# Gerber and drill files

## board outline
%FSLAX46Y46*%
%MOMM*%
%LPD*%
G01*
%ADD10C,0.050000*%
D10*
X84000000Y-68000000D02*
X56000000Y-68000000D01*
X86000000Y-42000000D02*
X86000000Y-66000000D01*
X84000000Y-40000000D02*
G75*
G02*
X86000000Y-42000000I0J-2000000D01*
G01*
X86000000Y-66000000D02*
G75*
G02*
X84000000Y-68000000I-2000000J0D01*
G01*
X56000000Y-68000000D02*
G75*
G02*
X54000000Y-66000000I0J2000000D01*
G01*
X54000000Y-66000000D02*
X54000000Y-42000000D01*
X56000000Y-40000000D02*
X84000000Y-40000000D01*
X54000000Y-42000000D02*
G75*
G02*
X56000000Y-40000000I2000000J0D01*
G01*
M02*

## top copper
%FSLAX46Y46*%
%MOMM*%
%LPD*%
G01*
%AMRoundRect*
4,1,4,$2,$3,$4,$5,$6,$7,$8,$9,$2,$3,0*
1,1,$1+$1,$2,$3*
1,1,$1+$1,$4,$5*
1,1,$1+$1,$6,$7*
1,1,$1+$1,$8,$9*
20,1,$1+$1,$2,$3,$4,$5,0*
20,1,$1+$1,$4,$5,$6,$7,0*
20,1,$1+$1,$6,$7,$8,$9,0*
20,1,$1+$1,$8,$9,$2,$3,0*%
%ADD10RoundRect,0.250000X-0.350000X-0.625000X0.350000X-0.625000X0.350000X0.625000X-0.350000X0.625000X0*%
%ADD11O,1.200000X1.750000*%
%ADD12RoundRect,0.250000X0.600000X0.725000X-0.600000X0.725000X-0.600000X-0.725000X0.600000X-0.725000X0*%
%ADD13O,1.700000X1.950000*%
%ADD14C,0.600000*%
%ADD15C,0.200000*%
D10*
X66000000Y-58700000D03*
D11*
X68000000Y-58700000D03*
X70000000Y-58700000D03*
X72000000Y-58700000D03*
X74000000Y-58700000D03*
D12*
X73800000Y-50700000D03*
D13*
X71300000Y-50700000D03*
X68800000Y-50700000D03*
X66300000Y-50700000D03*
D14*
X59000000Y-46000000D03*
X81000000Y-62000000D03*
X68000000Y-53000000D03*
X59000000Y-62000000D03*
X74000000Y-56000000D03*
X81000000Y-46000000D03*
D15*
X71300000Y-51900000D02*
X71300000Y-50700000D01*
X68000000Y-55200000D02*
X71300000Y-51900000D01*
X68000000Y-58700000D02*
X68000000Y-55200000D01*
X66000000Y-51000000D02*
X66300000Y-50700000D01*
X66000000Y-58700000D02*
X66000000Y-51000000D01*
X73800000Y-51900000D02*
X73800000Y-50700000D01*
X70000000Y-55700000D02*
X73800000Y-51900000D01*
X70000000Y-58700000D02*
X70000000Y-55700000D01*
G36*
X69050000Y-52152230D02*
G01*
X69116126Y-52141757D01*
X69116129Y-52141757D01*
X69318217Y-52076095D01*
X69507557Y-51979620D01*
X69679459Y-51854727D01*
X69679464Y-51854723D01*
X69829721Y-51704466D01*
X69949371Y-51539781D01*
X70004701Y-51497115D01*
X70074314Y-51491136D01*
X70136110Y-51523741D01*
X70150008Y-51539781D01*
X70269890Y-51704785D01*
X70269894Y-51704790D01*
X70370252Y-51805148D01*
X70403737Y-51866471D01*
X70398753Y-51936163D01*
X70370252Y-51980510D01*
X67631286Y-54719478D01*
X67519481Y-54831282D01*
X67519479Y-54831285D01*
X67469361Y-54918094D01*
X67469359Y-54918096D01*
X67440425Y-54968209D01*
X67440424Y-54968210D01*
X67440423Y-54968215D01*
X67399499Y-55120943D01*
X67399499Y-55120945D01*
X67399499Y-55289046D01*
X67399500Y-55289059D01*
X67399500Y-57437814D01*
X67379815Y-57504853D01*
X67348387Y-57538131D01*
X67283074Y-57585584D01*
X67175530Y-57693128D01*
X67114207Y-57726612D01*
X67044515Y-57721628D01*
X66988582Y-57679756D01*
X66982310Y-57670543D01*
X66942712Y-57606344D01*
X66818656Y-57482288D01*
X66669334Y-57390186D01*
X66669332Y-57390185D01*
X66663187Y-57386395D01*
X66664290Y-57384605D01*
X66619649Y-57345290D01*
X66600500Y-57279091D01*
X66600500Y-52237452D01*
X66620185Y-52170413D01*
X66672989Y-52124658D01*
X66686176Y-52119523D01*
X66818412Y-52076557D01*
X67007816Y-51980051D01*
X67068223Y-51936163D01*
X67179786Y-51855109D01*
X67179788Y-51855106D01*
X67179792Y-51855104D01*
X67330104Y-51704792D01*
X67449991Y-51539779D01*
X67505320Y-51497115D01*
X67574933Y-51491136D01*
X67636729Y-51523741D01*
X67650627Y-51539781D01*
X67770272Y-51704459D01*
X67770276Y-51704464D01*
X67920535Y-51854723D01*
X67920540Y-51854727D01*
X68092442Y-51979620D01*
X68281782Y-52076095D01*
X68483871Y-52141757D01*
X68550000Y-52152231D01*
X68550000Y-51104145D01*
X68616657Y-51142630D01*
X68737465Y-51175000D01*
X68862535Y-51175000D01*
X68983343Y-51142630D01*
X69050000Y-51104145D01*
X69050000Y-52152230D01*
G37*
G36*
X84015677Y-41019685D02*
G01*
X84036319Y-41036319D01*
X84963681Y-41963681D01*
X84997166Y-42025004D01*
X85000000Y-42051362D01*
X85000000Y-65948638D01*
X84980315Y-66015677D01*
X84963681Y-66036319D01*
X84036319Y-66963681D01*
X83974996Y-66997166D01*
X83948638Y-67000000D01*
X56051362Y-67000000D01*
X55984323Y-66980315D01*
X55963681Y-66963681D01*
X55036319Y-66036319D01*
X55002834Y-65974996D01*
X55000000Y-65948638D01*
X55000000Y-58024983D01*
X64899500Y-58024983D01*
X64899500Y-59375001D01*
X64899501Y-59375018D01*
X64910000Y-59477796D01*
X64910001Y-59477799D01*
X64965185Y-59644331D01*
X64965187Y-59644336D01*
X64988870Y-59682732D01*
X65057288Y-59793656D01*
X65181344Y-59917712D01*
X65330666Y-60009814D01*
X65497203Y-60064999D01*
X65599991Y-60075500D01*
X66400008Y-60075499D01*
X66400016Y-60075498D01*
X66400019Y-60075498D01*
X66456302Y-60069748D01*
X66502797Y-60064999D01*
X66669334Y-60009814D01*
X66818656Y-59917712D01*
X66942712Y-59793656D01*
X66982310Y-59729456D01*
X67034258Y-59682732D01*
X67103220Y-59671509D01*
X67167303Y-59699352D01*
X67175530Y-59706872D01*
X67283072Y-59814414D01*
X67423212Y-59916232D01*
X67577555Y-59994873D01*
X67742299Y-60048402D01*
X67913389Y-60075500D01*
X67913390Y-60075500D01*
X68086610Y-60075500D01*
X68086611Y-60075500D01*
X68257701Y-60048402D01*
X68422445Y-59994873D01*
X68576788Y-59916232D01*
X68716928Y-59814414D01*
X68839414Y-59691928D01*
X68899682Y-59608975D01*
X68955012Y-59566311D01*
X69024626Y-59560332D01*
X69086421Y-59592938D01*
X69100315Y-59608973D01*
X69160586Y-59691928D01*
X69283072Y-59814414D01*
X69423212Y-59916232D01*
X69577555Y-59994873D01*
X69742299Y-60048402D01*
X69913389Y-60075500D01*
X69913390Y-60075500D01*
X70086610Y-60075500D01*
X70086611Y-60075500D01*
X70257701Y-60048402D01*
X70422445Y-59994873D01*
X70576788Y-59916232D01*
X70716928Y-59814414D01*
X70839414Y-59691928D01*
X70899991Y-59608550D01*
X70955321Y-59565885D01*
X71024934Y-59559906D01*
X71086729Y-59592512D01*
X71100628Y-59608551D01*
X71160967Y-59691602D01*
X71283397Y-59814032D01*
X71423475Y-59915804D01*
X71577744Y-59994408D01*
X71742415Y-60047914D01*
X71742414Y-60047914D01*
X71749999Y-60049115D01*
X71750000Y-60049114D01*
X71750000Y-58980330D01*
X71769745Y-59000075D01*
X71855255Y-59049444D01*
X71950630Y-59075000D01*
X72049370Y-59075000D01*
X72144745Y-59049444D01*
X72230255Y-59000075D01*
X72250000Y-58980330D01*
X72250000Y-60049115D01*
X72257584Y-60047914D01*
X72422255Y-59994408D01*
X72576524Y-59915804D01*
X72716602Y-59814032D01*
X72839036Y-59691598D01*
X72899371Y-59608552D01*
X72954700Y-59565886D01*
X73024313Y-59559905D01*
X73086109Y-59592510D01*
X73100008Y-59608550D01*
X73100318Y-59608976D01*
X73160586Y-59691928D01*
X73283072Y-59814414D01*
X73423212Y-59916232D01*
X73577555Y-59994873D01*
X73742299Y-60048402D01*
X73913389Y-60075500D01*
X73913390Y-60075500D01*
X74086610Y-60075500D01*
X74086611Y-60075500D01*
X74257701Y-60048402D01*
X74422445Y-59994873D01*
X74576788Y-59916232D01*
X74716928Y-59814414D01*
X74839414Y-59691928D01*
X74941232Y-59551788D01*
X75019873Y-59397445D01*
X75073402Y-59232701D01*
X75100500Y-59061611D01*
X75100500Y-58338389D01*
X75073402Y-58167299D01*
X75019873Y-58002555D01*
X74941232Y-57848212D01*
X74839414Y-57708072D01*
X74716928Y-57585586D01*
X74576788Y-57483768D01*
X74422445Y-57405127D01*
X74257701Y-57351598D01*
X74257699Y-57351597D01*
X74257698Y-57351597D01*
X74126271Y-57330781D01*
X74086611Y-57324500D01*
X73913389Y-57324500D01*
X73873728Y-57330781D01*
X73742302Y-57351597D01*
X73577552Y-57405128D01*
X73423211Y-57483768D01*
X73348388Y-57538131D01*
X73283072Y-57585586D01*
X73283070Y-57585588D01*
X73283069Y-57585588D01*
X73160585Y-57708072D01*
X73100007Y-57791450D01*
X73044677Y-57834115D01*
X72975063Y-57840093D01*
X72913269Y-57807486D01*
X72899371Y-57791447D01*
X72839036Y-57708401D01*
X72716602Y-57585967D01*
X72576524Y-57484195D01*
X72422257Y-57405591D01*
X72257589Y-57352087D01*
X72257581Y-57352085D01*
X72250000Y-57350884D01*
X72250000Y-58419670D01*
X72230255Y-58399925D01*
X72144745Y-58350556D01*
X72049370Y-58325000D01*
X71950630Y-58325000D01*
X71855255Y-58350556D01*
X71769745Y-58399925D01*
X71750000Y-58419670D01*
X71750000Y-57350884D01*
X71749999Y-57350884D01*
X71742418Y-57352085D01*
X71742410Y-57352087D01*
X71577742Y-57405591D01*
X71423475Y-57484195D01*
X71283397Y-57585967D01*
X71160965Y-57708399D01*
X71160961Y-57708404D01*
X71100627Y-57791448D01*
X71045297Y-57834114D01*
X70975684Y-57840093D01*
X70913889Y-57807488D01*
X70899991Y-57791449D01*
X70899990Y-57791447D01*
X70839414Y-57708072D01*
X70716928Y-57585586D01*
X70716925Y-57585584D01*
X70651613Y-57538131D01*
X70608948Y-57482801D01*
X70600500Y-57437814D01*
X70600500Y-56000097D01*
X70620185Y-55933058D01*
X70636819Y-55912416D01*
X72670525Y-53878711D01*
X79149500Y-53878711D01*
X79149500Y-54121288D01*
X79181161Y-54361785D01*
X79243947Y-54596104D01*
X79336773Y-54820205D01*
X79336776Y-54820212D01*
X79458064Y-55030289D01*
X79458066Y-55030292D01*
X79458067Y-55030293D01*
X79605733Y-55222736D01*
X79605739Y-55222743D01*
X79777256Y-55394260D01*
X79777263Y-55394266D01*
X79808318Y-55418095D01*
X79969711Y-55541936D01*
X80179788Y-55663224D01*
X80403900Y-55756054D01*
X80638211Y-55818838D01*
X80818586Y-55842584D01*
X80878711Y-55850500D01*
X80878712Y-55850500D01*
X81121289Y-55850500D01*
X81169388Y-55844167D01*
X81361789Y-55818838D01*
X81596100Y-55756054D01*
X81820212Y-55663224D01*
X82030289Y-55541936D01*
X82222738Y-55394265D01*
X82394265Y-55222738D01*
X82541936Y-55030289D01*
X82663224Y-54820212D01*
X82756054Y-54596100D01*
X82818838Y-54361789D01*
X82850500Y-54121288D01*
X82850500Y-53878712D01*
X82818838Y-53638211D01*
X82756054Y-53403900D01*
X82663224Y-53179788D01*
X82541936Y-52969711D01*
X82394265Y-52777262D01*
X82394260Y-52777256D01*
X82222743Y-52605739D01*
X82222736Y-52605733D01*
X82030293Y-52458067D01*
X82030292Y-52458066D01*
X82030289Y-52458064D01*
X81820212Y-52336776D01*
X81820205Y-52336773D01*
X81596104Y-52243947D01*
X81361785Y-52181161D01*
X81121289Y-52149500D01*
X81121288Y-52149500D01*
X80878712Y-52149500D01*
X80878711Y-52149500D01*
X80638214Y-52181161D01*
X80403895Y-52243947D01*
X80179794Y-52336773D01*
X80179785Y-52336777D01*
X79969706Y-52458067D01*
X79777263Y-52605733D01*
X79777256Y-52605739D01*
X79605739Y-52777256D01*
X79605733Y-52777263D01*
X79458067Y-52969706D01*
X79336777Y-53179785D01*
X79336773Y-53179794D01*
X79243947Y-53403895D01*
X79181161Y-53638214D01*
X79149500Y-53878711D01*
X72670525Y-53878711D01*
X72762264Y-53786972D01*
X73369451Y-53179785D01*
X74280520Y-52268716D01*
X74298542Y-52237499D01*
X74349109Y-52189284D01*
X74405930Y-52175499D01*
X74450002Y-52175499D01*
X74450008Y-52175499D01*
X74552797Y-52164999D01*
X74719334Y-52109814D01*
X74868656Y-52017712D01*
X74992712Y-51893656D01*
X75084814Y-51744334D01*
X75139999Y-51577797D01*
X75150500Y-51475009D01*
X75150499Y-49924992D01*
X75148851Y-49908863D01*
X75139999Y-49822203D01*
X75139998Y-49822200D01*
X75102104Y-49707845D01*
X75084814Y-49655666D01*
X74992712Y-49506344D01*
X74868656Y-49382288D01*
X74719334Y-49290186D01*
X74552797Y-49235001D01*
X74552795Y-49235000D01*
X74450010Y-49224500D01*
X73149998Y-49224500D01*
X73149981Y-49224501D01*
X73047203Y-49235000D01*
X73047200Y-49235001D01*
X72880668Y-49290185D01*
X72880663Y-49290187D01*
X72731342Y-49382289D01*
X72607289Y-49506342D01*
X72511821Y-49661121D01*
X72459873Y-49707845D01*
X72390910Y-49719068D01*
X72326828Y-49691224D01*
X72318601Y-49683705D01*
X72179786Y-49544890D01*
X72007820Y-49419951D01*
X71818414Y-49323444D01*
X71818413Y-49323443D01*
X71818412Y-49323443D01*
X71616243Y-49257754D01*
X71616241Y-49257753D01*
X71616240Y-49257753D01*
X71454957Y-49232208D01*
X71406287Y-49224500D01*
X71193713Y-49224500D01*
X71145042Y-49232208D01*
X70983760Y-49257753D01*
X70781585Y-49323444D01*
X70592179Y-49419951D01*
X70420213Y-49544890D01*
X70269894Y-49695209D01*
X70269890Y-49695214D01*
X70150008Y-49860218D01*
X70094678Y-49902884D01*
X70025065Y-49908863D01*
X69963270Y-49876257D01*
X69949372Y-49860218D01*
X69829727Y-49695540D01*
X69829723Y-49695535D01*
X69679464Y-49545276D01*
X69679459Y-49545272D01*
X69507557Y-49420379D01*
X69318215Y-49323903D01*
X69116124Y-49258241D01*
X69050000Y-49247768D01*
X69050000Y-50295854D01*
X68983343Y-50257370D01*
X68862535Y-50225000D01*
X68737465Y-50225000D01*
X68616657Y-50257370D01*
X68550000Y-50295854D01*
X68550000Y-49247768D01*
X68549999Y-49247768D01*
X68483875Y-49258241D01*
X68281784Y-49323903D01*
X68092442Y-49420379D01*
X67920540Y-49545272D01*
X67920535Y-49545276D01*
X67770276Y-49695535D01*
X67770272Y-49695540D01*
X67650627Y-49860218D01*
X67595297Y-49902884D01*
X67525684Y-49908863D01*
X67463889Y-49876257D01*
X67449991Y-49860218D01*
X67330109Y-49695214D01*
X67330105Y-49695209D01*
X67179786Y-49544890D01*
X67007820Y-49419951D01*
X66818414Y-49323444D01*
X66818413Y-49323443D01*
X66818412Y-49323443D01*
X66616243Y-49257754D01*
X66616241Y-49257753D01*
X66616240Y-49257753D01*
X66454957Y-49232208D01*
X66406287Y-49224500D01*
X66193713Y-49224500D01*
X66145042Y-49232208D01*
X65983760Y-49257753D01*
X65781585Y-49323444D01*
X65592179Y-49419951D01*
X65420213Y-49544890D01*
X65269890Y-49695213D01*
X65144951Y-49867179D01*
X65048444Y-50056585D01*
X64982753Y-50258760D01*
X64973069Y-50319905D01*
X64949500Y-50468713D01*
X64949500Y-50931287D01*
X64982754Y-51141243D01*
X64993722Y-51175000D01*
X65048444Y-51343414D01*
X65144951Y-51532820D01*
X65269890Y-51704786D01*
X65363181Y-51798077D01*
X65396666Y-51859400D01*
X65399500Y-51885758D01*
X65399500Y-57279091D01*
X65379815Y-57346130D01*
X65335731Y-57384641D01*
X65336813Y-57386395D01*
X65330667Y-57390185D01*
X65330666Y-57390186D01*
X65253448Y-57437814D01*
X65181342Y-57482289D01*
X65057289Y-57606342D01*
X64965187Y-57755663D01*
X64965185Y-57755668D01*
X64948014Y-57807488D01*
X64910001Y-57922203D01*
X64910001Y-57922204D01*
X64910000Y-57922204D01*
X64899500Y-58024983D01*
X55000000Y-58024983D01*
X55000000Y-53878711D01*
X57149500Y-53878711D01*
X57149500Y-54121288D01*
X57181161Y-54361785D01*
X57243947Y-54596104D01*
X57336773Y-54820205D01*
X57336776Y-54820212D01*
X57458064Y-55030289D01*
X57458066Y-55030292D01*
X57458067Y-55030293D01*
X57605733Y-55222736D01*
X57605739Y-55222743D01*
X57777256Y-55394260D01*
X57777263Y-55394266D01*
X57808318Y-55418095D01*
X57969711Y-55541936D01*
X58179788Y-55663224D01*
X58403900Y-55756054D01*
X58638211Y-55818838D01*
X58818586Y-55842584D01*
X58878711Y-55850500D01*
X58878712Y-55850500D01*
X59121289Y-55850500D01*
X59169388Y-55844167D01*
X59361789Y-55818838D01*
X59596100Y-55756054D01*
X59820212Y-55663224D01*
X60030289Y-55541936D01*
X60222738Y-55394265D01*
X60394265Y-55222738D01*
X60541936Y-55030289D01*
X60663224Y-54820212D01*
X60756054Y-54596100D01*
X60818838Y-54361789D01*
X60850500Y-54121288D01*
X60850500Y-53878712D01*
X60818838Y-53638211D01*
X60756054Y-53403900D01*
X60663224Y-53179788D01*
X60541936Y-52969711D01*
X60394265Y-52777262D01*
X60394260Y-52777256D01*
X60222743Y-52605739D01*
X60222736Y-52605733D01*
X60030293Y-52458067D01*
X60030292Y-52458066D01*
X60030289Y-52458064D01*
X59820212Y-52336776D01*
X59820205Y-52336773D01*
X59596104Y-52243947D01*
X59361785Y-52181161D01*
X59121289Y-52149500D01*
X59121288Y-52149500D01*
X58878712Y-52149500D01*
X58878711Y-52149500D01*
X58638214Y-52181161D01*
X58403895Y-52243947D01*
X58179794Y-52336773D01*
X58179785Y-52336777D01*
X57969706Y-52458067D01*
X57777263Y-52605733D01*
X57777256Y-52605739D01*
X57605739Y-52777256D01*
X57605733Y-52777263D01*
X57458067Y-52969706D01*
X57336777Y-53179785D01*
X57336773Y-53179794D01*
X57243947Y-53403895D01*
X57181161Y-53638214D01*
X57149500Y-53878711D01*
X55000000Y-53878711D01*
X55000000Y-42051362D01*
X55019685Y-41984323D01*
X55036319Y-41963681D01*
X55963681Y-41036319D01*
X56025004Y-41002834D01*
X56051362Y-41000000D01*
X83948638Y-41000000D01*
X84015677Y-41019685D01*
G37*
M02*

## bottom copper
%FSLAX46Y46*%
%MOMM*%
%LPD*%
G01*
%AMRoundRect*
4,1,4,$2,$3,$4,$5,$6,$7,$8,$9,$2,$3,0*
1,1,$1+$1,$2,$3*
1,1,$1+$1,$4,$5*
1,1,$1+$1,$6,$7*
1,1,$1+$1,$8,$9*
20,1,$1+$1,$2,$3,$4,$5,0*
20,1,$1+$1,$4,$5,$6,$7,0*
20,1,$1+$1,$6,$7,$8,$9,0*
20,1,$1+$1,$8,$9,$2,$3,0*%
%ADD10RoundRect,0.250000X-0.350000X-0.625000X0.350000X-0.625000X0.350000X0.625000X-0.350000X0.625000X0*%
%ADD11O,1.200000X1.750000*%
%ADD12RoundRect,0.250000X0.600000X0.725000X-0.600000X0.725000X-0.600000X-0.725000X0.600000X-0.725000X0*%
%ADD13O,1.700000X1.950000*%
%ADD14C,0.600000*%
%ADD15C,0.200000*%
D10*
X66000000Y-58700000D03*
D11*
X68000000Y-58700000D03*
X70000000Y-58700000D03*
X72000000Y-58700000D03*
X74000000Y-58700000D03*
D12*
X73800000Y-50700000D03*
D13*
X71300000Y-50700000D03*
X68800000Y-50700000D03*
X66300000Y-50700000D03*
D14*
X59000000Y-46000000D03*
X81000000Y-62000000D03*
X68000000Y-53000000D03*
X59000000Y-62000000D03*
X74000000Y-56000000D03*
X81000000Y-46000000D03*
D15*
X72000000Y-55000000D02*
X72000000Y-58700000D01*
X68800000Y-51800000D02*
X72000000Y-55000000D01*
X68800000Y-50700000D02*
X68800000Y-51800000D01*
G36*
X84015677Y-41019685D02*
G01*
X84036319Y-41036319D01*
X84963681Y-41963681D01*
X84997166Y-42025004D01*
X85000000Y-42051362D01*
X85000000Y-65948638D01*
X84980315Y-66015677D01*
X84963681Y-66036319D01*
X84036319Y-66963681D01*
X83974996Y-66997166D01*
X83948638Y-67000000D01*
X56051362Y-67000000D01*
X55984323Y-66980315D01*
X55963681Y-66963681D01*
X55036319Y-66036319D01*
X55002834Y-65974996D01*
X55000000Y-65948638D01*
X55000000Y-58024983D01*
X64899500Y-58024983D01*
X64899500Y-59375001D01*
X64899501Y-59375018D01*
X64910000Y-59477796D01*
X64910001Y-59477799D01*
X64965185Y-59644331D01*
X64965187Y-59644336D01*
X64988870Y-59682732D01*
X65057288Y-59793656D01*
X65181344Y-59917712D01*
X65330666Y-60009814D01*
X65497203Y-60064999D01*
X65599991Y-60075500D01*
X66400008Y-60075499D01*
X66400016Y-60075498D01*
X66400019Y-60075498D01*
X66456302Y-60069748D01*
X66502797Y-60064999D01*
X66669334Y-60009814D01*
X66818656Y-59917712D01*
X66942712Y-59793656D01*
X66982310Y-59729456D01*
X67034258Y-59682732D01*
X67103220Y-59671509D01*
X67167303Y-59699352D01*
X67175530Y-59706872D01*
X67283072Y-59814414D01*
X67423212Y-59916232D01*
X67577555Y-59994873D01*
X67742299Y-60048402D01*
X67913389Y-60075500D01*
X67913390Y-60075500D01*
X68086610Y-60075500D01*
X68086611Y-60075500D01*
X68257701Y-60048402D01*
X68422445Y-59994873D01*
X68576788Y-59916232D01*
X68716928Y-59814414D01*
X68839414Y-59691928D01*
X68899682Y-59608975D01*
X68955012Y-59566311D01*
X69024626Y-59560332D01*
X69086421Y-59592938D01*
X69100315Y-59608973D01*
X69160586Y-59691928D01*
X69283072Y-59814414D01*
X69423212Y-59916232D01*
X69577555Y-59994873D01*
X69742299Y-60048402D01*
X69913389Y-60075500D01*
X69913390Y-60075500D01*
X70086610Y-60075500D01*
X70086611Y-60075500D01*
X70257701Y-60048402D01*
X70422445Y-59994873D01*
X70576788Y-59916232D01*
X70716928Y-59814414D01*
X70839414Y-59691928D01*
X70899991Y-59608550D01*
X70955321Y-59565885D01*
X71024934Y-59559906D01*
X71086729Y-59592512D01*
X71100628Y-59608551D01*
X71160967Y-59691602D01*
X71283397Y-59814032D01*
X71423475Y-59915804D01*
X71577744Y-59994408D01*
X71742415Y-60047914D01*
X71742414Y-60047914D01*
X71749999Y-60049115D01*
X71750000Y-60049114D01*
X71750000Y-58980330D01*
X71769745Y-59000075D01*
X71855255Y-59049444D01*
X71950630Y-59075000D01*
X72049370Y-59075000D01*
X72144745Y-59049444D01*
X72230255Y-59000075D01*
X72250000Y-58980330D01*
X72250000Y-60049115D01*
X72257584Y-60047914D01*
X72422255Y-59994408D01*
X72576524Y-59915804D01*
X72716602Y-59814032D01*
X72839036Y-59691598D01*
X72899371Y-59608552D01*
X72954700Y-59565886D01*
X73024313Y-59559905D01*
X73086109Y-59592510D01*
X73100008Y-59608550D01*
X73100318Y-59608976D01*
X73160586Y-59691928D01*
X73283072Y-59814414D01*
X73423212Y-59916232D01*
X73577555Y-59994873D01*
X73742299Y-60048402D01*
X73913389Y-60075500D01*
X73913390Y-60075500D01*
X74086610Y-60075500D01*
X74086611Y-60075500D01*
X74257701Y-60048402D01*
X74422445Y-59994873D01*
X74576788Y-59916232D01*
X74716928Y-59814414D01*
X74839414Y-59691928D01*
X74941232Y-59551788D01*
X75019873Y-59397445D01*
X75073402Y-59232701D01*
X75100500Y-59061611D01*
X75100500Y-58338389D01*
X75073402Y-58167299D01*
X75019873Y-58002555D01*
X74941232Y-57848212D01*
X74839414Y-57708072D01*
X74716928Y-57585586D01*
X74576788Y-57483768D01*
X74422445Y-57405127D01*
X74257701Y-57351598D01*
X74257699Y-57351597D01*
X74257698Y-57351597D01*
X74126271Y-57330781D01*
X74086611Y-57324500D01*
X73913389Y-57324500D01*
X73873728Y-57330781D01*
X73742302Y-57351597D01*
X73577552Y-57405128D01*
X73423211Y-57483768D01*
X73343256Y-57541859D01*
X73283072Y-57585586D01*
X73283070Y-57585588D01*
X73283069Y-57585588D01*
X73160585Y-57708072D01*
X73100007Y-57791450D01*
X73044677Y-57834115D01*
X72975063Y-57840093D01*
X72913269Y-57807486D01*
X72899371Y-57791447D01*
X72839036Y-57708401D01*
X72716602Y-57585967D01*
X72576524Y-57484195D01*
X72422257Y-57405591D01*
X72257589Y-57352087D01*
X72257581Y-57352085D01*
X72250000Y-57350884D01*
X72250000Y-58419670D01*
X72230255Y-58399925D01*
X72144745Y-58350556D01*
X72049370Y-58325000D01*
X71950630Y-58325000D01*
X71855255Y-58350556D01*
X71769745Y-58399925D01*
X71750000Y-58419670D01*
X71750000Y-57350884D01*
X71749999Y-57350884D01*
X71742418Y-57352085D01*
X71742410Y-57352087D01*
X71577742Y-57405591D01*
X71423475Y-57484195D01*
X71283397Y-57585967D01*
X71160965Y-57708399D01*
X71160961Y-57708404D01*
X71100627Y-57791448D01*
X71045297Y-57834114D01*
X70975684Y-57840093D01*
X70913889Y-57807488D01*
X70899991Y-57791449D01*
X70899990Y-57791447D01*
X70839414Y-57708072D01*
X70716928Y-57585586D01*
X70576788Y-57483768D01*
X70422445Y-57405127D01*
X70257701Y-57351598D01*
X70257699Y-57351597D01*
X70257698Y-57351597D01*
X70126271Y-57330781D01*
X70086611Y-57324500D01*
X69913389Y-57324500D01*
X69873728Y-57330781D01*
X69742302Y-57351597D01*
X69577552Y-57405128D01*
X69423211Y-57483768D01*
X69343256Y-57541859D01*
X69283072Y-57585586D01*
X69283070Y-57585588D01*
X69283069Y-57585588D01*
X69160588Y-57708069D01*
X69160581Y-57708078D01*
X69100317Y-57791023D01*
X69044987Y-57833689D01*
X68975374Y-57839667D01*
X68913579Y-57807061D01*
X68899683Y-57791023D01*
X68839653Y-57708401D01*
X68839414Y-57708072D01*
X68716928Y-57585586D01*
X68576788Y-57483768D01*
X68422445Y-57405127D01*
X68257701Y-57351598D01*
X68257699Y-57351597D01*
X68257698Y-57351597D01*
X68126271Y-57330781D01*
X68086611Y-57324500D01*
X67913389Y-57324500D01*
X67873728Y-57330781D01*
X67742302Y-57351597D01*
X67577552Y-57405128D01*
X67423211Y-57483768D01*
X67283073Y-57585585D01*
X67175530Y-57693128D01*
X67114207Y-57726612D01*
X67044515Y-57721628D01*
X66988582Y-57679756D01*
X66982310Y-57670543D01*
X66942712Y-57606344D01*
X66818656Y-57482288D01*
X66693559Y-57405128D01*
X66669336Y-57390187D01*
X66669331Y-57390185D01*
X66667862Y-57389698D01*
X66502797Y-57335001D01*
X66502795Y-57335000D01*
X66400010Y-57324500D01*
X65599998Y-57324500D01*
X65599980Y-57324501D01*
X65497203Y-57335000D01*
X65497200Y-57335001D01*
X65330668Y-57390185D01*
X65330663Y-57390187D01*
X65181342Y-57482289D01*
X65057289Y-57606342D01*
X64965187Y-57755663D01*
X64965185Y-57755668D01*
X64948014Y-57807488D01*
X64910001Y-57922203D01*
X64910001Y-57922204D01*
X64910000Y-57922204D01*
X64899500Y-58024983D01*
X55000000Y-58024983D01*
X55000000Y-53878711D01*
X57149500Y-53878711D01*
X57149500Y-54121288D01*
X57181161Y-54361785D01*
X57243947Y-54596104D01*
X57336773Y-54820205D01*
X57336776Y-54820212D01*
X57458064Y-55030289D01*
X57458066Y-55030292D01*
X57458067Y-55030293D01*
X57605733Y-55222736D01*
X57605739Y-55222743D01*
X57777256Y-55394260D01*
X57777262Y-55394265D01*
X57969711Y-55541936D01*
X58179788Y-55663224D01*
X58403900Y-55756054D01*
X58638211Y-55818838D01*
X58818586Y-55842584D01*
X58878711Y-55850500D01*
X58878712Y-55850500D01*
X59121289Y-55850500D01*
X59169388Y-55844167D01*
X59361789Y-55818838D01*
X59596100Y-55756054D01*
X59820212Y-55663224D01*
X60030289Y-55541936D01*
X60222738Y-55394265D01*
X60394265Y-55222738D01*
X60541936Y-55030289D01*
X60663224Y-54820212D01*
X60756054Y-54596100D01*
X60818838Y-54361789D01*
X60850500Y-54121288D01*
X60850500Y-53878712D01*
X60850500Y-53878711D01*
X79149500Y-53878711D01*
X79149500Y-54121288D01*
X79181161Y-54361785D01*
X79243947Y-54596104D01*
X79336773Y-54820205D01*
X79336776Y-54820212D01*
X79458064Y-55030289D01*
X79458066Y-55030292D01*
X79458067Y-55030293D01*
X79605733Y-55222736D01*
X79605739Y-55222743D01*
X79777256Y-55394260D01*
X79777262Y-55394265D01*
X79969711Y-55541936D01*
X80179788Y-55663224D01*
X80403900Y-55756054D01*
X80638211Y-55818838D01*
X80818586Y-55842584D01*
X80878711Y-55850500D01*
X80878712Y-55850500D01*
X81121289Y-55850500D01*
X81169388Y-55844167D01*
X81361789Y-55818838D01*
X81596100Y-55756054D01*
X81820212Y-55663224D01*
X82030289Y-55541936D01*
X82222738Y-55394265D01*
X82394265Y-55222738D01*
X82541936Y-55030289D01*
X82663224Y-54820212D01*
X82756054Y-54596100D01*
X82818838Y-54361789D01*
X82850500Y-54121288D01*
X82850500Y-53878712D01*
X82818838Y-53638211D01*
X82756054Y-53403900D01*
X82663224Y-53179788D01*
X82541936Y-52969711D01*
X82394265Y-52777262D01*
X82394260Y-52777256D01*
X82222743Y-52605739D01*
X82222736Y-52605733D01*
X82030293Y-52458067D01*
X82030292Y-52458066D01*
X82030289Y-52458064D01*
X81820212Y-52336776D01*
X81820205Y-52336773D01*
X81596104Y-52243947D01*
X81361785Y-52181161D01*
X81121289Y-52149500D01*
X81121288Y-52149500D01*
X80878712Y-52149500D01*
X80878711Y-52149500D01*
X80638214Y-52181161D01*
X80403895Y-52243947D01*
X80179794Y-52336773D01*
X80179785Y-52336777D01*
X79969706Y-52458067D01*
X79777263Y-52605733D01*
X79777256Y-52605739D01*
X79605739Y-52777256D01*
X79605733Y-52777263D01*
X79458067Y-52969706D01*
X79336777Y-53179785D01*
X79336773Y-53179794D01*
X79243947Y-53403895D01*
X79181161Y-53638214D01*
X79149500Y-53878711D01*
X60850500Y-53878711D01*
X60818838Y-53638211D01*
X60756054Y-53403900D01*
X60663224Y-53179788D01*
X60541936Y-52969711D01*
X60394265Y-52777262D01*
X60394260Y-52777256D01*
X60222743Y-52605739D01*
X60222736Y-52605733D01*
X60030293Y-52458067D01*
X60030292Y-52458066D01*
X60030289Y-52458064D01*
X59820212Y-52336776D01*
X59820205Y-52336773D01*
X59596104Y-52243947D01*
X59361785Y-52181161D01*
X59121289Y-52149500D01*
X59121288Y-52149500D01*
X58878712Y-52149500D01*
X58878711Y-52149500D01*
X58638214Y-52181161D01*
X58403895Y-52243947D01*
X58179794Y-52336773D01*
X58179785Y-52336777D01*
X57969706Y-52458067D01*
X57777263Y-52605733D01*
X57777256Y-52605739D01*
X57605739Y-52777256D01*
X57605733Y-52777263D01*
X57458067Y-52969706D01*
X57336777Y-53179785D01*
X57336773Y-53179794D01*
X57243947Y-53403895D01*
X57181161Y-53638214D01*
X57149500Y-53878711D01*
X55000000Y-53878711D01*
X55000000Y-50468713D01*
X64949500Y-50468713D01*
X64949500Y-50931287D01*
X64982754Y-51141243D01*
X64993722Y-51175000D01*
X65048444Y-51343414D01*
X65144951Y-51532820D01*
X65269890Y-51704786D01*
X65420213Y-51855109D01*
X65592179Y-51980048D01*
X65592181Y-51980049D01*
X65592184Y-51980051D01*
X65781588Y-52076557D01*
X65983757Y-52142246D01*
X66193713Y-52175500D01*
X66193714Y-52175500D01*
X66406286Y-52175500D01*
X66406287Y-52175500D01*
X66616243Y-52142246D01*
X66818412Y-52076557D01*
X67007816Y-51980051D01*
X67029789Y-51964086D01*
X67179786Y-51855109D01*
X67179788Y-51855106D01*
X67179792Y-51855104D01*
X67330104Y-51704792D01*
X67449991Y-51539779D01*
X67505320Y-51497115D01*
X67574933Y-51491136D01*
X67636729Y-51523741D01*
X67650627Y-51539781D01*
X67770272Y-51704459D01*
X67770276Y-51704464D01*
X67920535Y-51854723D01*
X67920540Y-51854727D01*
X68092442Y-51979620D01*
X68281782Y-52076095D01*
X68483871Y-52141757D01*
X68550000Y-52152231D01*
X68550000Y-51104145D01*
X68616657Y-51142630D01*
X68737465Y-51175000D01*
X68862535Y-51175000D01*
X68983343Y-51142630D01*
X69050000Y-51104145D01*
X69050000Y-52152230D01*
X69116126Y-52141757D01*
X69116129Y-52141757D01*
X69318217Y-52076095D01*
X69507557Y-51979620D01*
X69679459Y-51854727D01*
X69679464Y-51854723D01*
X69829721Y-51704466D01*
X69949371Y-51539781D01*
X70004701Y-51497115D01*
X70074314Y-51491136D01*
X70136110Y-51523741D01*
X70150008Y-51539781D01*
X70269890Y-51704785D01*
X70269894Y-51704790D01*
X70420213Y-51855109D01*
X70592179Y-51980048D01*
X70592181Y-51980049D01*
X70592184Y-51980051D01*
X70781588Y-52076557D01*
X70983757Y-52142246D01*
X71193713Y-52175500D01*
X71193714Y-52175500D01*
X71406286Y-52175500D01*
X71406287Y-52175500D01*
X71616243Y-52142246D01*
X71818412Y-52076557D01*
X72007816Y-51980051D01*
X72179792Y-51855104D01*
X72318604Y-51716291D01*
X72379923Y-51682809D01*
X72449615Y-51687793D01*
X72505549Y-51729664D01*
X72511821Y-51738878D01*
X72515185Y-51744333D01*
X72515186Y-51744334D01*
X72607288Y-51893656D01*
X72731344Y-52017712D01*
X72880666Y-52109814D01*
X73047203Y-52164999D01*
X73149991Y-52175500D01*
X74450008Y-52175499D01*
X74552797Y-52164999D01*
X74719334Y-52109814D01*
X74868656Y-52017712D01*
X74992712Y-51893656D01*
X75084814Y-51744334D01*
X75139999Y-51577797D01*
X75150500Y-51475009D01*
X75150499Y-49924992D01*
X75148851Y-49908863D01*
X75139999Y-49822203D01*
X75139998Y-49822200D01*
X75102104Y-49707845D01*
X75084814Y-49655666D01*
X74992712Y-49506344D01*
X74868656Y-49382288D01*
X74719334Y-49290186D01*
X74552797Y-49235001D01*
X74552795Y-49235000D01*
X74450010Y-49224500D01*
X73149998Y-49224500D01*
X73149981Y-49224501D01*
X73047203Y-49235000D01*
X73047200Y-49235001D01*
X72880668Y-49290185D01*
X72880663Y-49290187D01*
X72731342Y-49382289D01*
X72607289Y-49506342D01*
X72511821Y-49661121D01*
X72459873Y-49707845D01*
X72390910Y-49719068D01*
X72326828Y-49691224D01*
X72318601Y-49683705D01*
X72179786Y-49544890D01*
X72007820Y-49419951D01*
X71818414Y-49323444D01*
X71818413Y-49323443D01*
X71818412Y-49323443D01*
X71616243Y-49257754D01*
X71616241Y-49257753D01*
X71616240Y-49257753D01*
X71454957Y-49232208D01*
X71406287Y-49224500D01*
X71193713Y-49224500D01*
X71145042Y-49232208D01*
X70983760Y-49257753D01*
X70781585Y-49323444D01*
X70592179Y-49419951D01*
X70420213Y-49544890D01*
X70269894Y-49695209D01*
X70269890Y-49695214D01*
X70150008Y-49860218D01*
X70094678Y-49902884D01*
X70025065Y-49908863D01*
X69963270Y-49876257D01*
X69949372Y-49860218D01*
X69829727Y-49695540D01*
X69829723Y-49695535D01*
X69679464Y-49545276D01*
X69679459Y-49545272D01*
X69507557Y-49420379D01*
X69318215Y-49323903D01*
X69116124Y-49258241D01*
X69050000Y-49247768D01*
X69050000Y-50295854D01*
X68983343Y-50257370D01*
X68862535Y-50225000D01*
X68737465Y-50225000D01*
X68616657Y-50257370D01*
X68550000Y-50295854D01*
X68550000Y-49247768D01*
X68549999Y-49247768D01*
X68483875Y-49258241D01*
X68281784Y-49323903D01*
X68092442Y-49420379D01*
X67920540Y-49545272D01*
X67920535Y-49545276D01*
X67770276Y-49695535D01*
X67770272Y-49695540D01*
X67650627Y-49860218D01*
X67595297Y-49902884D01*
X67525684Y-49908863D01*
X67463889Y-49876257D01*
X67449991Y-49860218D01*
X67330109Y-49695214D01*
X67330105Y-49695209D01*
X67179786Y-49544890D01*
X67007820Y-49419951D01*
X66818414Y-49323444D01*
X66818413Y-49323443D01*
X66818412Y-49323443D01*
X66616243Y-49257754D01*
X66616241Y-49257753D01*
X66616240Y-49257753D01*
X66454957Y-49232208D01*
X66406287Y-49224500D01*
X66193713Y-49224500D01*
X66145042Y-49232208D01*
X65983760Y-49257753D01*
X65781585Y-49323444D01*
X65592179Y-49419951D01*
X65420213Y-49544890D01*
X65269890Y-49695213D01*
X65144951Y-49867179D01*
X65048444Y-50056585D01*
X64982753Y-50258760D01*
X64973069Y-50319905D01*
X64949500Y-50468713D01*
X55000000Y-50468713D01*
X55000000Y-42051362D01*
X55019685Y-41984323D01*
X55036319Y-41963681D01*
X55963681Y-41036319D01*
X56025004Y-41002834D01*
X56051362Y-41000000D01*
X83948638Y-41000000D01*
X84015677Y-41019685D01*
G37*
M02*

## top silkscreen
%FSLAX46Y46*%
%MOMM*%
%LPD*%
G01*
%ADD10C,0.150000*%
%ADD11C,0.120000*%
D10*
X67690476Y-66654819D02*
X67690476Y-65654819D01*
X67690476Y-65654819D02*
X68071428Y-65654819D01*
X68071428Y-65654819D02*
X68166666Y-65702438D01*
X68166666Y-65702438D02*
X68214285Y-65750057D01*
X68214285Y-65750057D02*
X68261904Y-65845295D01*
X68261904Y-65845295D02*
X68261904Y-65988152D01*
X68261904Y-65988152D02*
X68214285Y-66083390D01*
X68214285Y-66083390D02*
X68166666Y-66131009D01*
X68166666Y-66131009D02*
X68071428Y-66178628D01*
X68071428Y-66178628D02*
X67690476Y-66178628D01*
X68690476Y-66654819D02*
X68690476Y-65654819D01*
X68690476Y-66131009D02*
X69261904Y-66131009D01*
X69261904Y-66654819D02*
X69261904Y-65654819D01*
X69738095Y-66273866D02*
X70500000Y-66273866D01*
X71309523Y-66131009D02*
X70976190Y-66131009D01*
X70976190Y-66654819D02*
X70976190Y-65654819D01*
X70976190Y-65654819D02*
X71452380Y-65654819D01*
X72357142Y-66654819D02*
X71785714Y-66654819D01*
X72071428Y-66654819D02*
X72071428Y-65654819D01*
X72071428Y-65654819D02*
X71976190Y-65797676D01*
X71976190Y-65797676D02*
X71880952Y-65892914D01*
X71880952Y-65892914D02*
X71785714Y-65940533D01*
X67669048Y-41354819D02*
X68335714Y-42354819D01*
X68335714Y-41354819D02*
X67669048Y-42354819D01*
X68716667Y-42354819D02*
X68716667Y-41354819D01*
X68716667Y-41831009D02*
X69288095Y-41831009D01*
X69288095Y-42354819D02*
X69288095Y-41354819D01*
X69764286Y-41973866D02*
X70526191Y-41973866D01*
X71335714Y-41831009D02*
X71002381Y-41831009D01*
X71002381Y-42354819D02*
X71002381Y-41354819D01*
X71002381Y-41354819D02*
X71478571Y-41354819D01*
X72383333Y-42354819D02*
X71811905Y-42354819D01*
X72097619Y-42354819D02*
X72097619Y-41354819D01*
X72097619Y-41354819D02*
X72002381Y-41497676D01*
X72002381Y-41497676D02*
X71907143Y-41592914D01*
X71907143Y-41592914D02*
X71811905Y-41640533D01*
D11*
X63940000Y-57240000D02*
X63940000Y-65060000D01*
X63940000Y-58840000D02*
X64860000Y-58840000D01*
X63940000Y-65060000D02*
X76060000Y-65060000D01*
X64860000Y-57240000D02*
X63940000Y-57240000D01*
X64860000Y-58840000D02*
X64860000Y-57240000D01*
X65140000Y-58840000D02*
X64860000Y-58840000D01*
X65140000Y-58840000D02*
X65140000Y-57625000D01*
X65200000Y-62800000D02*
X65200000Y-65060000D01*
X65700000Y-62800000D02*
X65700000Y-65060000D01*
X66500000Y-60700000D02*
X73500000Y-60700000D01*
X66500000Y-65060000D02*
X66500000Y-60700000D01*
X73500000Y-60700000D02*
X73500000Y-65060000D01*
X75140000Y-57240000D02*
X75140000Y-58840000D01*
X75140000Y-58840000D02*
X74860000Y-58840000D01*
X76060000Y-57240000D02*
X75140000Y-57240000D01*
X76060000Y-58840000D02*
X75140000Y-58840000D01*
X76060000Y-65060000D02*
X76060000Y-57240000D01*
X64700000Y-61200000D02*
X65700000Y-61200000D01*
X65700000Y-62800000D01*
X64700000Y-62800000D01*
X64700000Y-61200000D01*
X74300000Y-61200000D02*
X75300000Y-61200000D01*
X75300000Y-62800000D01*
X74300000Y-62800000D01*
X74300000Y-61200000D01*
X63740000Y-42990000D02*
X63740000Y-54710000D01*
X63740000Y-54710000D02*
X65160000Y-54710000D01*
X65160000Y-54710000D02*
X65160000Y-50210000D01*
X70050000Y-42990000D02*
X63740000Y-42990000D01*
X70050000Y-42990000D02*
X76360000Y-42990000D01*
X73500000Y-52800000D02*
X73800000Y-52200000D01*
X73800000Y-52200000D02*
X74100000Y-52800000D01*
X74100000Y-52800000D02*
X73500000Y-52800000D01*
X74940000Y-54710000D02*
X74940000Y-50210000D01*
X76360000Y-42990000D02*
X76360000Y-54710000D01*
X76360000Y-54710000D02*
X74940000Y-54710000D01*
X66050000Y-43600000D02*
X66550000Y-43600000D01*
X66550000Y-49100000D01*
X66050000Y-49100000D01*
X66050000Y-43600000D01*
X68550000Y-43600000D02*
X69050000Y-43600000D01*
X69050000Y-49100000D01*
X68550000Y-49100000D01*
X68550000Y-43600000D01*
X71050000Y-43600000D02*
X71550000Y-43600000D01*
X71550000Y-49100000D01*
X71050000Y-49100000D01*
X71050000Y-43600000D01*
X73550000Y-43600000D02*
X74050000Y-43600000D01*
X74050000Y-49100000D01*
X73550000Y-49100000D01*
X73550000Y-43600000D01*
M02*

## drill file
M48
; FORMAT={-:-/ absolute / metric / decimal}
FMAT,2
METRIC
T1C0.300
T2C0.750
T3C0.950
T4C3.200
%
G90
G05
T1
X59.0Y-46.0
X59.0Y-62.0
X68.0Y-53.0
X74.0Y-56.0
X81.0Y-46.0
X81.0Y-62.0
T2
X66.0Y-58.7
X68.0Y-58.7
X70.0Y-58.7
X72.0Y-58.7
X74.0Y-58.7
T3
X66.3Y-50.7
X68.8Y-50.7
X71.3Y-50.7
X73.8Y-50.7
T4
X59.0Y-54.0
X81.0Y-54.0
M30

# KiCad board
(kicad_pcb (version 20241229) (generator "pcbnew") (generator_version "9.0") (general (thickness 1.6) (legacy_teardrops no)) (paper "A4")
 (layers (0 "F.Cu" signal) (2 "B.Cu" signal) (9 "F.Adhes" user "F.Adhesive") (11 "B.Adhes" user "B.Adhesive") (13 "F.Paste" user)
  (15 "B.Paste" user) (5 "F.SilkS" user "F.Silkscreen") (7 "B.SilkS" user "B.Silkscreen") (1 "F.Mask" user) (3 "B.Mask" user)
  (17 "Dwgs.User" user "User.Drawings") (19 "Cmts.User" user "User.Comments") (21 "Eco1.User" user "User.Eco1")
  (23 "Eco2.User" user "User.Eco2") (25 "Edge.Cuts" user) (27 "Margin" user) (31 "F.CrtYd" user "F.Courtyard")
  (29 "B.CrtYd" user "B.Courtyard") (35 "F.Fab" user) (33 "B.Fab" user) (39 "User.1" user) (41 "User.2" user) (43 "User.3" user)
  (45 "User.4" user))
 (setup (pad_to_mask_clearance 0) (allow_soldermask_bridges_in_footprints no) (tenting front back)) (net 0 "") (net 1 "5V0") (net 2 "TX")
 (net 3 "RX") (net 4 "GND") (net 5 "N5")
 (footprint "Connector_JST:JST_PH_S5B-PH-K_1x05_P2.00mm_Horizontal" (layer "F.Cu") (at 66 58.7)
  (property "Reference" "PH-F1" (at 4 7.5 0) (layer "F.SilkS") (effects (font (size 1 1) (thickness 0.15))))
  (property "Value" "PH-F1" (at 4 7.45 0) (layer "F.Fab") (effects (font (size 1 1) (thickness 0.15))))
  (fp_line (start -2.06 -1.46) (end -2.06 6.36) (stroke (width 0.12) (type solid)) (layer "F.SilkS"))
  (fp_line (start -2.06 0.14) (end -1.14 0.14) (stroke (width 0.12) (type solid)) (layer "F.SilkS"))
  (fp_line (start -2.06 6.36) (end 10.06 6.36) (stroke (width 0.12) (type solid)) (layer "F.SilkS"))
  (fp_line (start -1.14 -1.46) (end -2.06 -1.46) (stroke (width 0.12) (type solid)) (layer "F.SilkS"))
  (fp_line (start -1.14 0.14) (end -1.14 -1.46) (stroke (width 0.12) (type solid)) (layer "F.SilkS"))
  (fp_line (start -0.86 0.14) (end -1.14 0.14) (stroke (width 0.12) (type solid)) (layer "F.SilkS"))
  (fp_line (start -0.86 0.14) (end -0.86 -1.075) (stroke (width 0.12) (type solid)) (layer "F.SilkS"))
  (fp_line (start -0.8 4.1) (end -0.8 6.36) (stroke (width 0.12) (type solid)) (layer "F.SilkS"))
  (fp_line (start -0.3 4.1) (end -0.3 6.36) (stroke (width 0.12) (type solid)) (layer "F.SilkS"))
  (fp_line (start 0.5 2) (end 7.5 2) (stroke (width 0.12) (type solid)) (layer "F.SilkS"))
  (fp_line (start 0.5 6.36) (end 0.5 2) (stroke (width 0.12) (type solid)) (layer "F.SilkS"))
  (fp_line (start 7.5 2) (end 7.5 6.36) (stroke (width 0.12) (type solid)) (layer "F.SilkS"))
  (fp_line (start 9.14 -1.46) (end 9.14 0.14) (stroke (width 0.12) (type solid)) (layer "F.SilkS"))
  (fp_line (start 9.14 0.14) (end 8.86 0.14) (stroke (width 0.12) (type solid)) (layer "F.SilkS"))
  (fp_line (start 10.06 -1.46) (end 9.14 -1.46) (stroke (width 0.12) (type solid)) (layer "F.SilkS"))
  (fp_line (start 10.06 0.14) (end 9.14 0.14) (stroke (width 0.12) (type solid)) (layer "F.SilkS"))
  (fp_line (start 10.06 6.36) (end 10.06 -1.46) (stroke (width 0.12) (type solid)) (layer "F.SilkS"))
  (fp_rect (start -1.3 2.5) (end -0.3 4.1) (stroke (width 0.12) (type solid)) (fill no) (layer "F.SilkS"))
  (fp_rect (start 8.3 2.5) (end 9.3 4.1) (stroke (width 0.12) (type solid)) (fill no) (layer "F.SilkS"))
  (pad "1" thru_hole roundrect (at 0 0) (size 1.2 1.75) (drill 0.75) (layers "*.Cu" "*.Mask") (remove_unused_layers no)
   (roundrect_rratio 0.208333) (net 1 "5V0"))
  (pad "2" thru_hole oval (at 2 0) (size 1.2 1.75) (drill 0.75) (layers "*.Cu" "*.Mask") (remove_unused_layers no) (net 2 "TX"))
  (pad "3" thru_hole oval (at 4 0) (size 1.2 1.75) (drill 0.75) (layers "*.Cu" "*.Mask") (remove_unused_layers no) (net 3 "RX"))
  (pad "4" thru_hole oval (at 6 0) (size 1.2 1.75) (drill 0.75) (layers "*.Cu" "*.Mask") (remove_unused_layers no) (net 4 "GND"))
  (pad "5" thru_hole oval (at 8 0) (size 1.2 1.75) (drill 0.75) (layers "*.Cu" "*.Mask") (remove_unused_layers no) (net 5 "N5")))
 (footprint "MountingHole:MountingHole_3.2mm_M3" (layer "F.Cu") (at 59 54)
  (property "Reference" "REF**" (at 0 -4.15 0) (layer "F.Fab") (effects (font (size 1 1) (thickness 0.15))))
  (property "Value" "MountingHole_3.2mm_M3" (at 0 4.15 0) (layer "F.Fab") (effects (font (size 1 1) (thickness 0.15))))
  (pad "" np_thru_hole circle (at 0 0) (size 3.2 3.2) (drill 3.2) (layers "*.Cu" "*.Mask")))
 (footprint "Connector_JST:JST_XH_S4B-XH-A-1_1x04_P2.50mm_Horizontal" (layer "F.Cu") (at 73.8 50.7 180)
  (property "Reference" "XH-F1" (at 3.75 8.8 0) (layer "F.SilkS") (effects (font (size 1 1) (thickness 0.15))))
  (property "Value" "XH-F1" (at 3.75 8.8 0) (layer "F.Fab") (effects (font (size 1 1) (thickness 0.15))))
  (fp_line (start 10.06 7.71) (end 10.06 -4.01) (stroke (width 0.12) (type solid)) (layer "F.SilkS"))
  (fp_line (start 10.06 -4.01) (end 8.64 -4.01) (stroke (width 0.12) (type solid)) (layer "F.SilkS"))
  (fp_line (start 8.64 -4.01) (end 8.64 0.49) (stroke (width 0.12) (type solid)) (layer "F.SilkS"))
  (fp_line (start 3.75 7.71) (end 10.06 7.71) (stroke (width 0.12) (type solid)) (layer "F.SilkS"))
  (fp_line (start 3.75 7.71) (end -2.56 7.71) (stroke (width 0.12) (type solid)) (layer "F.SilkS"))
  (fp_line (start 0.3 -2.1) (end 0 -1.5) (stroke (width 0.12) (type solid)) (layer "F.SilkS"))
  (fp_line (start 0 -1.5) (end -0.3 -2.1) (stroke (width 0.12) (type solid)) (layer "F.SilkS"))
  (fp_line (start -0.3 -2.1) (end 0.3 -2.1) (stroke (width 0.12) (type solid)) (layer "F.SilkS"))
  (fp_line (start -1.14 -4.01) (end -1.14 0.49) (stroke (width 0.12) (type solid)) (layer "F.SilkS"))
  (fp_line (start -2.56 7.71) (end -2.56 -4.01) (stroke (width 0.12) (type solid)) (layer "F.SilkS"))
  (fp_line (start -2.56 -4.01) (end -1.14 -4.01) (stroke (width 0.12) (type solid)) (layer "F.SilkS"))
  (fp_rect (start 7.25 1.6) (end 7.75 7.1) (stroke (width 0.12) (type solid)) (fill no) (layer "F.SilkS"))
  (fp_rect (start 4.75 1.6) (end 5.25 7.1) (stroke (width 0.12) (type solid)) (fill no) (layer "F.SilkS"))
  (fp_rect (start 2.25 1.6) (end 2.75 7.1) (stroke (width 0.12) (type solid)) (fill no) (layer "F.SilkS"))
  (fp_rect (start -0.25 1.6) (end 0.25 7.1) (stroke (width 0.12) (type solid)) (fill no) (layer "F.SilkS"))
  (pad "1" thru_hole roundrect (at 0 0 180) (size 1.7 1.95) (drill 0.95) (layers "*.Cu" "*.Mask") (remove_unused_layers no)
   (roundrect_rratio 0.147059) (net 3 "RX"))
  (pad "2" thru_hole oval (at 2.5 0 180) (size 1.7 1.95) (drill 0.95) (layers "*.Cu" "*.Mask") (remove_unused_layers no) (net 2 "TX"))
  (pad "3" thru_hole oval (at 5 0 180) (size 1.7 1.95) (drill 0.95) (layers "*.Cu" "*.Mask") (remove_unused_layers no) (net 4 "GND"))
  (pad "4" thru_hole oval (at 7.5 0 180) (size 1.7 1.95) (drill 0.95) (layers "*.Cu" "*.Mask") (remove_unused_layers no) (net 1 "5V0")))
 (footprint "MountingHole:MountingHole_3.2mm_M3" (layer "F.Cu") (at 81 54)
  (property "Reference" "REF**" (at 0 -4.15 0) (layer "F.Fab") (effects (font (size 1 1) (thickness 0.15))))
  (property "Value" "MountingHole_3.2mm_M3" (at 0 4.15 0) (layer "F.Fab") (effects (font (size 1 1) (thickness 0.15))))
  (pad "" np_thru_hole circle (at 0 0) (size 3.2 3.2) (drill 3.2) (layers "*.Cu" "*.Mask")))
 (gr_line (start 84 68) (end 56 68) (stroke (width 0.05) (type default)) (layer "Edge.Cuts"))
 (gr_line (start 86 42) (end 86 66) (stroke (width 0.05) (type default)) (layer "Edge.Cuts"))
 (gr_arc (start 84 40) (mid 85.414214 40.585786) (end 86 42) (stroke (width 0.05) (type default)) (layer "Edge.Cuts"))
 (gr_arc (start 86 66) (mid 85.414214 67.414214) (end 84 68) (stroke (width 0.05) (type default)) (layer "Edge.Cuts"))
 (gr_arc (start 56 68) (mid 54.585786 67.414214) (end 54 66) (stroke (width 0.05) (type default)) (layer "Edge.Cuts"))
 (gr_line (start 54 66) (end 54 42) (stroke (width 0.05) (type default)) (layer "Edge.Cuts"))
 (gr_line (start 56 40) (end 84 40) (stroke (width 0.05) (type default)) (layer "Edge.Cuts"))
 (gr_arc (start 54 42) (mid 54.585786 40.585786) (end 56 40) (stroke (width 0.05) (type default)) (layer "Edge.Cuts"))
 (segment (start 71.3 51.9) (end 71.3 50.7) (width 0.2) (layer "F.Cu") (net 2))
 (segment (start 68 55.2) (end 71.3 51.9) (width 0.2) (layer "F.Cu") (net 2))
 (segment (start 68 58.7) (end 68 55.2) (width 0.2) (layer "F.Cu") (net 2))
 (segment (start 66 51) (end 66.3 50.7) (width 0.2) (layer "F.Cu") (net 1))
 (segment (start 66 58.7) (end 66 51) (width 0.2) (layer "F.Cu") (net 1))
 (segment (start 73.8 51.9) (end 73.8 50.7) (width 0.2) (layer "F.Cu") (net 3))
 (segment (start 70 55.7) (end 73.8 51.9) (width 0.2) (layer "F.Cu") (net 3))
 (segment (start 70 58.7) (end 70 55.7) (width 0.2) (layer "F.Cu") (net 3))
 (via (at 59 46) (size 0.6) (drill 0.3) (layers "F.Cu" "B.Cu") (free yes) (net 4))
 (via (at 81 62) (size 0.6) (drill 0.3) (layers "F.Cu" "B.Cu") (free yes) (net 4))
 (via (at 68 53) (size 0.6) (drill 0.3) (layers "F.Cu" "B.Cu") (free yes) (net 4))
 (via (at 59 62) (size 0.6) (drill 0.3) (layers "F.Cu" "B.Cu") (free yes) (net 4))
 (via (at 74 56) (size 0.6) (drill 0.3) (layers "F.Cu" "B.Cu") (free yes) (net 4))
 (via (at 81 46) (size 0.6) (drill 0.3) (layers "F.Cu" "B.Cu") (free yes) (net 4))
 (segment (start 72 55) (end 72 58.7) (width 0.2) (layer "B.Cu") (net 4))
 (segment (start 68.8 51.8) (end 72 55) (width 0.2) (layer "B.Cu") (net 4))
 (segment (start 68.8 50.7) (end 68.8 51.8) (width 0.2) (layer "B.Cu") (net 4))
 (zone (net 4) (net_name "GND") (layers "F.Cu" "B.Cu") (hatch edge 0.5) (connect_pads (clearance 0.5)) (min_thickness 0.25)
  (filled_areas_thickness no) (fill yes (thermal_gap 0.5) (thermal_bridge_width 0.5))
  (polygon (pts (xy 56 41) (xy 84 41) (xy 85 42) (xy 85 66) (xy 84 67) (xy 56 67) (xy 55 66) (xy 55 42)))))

